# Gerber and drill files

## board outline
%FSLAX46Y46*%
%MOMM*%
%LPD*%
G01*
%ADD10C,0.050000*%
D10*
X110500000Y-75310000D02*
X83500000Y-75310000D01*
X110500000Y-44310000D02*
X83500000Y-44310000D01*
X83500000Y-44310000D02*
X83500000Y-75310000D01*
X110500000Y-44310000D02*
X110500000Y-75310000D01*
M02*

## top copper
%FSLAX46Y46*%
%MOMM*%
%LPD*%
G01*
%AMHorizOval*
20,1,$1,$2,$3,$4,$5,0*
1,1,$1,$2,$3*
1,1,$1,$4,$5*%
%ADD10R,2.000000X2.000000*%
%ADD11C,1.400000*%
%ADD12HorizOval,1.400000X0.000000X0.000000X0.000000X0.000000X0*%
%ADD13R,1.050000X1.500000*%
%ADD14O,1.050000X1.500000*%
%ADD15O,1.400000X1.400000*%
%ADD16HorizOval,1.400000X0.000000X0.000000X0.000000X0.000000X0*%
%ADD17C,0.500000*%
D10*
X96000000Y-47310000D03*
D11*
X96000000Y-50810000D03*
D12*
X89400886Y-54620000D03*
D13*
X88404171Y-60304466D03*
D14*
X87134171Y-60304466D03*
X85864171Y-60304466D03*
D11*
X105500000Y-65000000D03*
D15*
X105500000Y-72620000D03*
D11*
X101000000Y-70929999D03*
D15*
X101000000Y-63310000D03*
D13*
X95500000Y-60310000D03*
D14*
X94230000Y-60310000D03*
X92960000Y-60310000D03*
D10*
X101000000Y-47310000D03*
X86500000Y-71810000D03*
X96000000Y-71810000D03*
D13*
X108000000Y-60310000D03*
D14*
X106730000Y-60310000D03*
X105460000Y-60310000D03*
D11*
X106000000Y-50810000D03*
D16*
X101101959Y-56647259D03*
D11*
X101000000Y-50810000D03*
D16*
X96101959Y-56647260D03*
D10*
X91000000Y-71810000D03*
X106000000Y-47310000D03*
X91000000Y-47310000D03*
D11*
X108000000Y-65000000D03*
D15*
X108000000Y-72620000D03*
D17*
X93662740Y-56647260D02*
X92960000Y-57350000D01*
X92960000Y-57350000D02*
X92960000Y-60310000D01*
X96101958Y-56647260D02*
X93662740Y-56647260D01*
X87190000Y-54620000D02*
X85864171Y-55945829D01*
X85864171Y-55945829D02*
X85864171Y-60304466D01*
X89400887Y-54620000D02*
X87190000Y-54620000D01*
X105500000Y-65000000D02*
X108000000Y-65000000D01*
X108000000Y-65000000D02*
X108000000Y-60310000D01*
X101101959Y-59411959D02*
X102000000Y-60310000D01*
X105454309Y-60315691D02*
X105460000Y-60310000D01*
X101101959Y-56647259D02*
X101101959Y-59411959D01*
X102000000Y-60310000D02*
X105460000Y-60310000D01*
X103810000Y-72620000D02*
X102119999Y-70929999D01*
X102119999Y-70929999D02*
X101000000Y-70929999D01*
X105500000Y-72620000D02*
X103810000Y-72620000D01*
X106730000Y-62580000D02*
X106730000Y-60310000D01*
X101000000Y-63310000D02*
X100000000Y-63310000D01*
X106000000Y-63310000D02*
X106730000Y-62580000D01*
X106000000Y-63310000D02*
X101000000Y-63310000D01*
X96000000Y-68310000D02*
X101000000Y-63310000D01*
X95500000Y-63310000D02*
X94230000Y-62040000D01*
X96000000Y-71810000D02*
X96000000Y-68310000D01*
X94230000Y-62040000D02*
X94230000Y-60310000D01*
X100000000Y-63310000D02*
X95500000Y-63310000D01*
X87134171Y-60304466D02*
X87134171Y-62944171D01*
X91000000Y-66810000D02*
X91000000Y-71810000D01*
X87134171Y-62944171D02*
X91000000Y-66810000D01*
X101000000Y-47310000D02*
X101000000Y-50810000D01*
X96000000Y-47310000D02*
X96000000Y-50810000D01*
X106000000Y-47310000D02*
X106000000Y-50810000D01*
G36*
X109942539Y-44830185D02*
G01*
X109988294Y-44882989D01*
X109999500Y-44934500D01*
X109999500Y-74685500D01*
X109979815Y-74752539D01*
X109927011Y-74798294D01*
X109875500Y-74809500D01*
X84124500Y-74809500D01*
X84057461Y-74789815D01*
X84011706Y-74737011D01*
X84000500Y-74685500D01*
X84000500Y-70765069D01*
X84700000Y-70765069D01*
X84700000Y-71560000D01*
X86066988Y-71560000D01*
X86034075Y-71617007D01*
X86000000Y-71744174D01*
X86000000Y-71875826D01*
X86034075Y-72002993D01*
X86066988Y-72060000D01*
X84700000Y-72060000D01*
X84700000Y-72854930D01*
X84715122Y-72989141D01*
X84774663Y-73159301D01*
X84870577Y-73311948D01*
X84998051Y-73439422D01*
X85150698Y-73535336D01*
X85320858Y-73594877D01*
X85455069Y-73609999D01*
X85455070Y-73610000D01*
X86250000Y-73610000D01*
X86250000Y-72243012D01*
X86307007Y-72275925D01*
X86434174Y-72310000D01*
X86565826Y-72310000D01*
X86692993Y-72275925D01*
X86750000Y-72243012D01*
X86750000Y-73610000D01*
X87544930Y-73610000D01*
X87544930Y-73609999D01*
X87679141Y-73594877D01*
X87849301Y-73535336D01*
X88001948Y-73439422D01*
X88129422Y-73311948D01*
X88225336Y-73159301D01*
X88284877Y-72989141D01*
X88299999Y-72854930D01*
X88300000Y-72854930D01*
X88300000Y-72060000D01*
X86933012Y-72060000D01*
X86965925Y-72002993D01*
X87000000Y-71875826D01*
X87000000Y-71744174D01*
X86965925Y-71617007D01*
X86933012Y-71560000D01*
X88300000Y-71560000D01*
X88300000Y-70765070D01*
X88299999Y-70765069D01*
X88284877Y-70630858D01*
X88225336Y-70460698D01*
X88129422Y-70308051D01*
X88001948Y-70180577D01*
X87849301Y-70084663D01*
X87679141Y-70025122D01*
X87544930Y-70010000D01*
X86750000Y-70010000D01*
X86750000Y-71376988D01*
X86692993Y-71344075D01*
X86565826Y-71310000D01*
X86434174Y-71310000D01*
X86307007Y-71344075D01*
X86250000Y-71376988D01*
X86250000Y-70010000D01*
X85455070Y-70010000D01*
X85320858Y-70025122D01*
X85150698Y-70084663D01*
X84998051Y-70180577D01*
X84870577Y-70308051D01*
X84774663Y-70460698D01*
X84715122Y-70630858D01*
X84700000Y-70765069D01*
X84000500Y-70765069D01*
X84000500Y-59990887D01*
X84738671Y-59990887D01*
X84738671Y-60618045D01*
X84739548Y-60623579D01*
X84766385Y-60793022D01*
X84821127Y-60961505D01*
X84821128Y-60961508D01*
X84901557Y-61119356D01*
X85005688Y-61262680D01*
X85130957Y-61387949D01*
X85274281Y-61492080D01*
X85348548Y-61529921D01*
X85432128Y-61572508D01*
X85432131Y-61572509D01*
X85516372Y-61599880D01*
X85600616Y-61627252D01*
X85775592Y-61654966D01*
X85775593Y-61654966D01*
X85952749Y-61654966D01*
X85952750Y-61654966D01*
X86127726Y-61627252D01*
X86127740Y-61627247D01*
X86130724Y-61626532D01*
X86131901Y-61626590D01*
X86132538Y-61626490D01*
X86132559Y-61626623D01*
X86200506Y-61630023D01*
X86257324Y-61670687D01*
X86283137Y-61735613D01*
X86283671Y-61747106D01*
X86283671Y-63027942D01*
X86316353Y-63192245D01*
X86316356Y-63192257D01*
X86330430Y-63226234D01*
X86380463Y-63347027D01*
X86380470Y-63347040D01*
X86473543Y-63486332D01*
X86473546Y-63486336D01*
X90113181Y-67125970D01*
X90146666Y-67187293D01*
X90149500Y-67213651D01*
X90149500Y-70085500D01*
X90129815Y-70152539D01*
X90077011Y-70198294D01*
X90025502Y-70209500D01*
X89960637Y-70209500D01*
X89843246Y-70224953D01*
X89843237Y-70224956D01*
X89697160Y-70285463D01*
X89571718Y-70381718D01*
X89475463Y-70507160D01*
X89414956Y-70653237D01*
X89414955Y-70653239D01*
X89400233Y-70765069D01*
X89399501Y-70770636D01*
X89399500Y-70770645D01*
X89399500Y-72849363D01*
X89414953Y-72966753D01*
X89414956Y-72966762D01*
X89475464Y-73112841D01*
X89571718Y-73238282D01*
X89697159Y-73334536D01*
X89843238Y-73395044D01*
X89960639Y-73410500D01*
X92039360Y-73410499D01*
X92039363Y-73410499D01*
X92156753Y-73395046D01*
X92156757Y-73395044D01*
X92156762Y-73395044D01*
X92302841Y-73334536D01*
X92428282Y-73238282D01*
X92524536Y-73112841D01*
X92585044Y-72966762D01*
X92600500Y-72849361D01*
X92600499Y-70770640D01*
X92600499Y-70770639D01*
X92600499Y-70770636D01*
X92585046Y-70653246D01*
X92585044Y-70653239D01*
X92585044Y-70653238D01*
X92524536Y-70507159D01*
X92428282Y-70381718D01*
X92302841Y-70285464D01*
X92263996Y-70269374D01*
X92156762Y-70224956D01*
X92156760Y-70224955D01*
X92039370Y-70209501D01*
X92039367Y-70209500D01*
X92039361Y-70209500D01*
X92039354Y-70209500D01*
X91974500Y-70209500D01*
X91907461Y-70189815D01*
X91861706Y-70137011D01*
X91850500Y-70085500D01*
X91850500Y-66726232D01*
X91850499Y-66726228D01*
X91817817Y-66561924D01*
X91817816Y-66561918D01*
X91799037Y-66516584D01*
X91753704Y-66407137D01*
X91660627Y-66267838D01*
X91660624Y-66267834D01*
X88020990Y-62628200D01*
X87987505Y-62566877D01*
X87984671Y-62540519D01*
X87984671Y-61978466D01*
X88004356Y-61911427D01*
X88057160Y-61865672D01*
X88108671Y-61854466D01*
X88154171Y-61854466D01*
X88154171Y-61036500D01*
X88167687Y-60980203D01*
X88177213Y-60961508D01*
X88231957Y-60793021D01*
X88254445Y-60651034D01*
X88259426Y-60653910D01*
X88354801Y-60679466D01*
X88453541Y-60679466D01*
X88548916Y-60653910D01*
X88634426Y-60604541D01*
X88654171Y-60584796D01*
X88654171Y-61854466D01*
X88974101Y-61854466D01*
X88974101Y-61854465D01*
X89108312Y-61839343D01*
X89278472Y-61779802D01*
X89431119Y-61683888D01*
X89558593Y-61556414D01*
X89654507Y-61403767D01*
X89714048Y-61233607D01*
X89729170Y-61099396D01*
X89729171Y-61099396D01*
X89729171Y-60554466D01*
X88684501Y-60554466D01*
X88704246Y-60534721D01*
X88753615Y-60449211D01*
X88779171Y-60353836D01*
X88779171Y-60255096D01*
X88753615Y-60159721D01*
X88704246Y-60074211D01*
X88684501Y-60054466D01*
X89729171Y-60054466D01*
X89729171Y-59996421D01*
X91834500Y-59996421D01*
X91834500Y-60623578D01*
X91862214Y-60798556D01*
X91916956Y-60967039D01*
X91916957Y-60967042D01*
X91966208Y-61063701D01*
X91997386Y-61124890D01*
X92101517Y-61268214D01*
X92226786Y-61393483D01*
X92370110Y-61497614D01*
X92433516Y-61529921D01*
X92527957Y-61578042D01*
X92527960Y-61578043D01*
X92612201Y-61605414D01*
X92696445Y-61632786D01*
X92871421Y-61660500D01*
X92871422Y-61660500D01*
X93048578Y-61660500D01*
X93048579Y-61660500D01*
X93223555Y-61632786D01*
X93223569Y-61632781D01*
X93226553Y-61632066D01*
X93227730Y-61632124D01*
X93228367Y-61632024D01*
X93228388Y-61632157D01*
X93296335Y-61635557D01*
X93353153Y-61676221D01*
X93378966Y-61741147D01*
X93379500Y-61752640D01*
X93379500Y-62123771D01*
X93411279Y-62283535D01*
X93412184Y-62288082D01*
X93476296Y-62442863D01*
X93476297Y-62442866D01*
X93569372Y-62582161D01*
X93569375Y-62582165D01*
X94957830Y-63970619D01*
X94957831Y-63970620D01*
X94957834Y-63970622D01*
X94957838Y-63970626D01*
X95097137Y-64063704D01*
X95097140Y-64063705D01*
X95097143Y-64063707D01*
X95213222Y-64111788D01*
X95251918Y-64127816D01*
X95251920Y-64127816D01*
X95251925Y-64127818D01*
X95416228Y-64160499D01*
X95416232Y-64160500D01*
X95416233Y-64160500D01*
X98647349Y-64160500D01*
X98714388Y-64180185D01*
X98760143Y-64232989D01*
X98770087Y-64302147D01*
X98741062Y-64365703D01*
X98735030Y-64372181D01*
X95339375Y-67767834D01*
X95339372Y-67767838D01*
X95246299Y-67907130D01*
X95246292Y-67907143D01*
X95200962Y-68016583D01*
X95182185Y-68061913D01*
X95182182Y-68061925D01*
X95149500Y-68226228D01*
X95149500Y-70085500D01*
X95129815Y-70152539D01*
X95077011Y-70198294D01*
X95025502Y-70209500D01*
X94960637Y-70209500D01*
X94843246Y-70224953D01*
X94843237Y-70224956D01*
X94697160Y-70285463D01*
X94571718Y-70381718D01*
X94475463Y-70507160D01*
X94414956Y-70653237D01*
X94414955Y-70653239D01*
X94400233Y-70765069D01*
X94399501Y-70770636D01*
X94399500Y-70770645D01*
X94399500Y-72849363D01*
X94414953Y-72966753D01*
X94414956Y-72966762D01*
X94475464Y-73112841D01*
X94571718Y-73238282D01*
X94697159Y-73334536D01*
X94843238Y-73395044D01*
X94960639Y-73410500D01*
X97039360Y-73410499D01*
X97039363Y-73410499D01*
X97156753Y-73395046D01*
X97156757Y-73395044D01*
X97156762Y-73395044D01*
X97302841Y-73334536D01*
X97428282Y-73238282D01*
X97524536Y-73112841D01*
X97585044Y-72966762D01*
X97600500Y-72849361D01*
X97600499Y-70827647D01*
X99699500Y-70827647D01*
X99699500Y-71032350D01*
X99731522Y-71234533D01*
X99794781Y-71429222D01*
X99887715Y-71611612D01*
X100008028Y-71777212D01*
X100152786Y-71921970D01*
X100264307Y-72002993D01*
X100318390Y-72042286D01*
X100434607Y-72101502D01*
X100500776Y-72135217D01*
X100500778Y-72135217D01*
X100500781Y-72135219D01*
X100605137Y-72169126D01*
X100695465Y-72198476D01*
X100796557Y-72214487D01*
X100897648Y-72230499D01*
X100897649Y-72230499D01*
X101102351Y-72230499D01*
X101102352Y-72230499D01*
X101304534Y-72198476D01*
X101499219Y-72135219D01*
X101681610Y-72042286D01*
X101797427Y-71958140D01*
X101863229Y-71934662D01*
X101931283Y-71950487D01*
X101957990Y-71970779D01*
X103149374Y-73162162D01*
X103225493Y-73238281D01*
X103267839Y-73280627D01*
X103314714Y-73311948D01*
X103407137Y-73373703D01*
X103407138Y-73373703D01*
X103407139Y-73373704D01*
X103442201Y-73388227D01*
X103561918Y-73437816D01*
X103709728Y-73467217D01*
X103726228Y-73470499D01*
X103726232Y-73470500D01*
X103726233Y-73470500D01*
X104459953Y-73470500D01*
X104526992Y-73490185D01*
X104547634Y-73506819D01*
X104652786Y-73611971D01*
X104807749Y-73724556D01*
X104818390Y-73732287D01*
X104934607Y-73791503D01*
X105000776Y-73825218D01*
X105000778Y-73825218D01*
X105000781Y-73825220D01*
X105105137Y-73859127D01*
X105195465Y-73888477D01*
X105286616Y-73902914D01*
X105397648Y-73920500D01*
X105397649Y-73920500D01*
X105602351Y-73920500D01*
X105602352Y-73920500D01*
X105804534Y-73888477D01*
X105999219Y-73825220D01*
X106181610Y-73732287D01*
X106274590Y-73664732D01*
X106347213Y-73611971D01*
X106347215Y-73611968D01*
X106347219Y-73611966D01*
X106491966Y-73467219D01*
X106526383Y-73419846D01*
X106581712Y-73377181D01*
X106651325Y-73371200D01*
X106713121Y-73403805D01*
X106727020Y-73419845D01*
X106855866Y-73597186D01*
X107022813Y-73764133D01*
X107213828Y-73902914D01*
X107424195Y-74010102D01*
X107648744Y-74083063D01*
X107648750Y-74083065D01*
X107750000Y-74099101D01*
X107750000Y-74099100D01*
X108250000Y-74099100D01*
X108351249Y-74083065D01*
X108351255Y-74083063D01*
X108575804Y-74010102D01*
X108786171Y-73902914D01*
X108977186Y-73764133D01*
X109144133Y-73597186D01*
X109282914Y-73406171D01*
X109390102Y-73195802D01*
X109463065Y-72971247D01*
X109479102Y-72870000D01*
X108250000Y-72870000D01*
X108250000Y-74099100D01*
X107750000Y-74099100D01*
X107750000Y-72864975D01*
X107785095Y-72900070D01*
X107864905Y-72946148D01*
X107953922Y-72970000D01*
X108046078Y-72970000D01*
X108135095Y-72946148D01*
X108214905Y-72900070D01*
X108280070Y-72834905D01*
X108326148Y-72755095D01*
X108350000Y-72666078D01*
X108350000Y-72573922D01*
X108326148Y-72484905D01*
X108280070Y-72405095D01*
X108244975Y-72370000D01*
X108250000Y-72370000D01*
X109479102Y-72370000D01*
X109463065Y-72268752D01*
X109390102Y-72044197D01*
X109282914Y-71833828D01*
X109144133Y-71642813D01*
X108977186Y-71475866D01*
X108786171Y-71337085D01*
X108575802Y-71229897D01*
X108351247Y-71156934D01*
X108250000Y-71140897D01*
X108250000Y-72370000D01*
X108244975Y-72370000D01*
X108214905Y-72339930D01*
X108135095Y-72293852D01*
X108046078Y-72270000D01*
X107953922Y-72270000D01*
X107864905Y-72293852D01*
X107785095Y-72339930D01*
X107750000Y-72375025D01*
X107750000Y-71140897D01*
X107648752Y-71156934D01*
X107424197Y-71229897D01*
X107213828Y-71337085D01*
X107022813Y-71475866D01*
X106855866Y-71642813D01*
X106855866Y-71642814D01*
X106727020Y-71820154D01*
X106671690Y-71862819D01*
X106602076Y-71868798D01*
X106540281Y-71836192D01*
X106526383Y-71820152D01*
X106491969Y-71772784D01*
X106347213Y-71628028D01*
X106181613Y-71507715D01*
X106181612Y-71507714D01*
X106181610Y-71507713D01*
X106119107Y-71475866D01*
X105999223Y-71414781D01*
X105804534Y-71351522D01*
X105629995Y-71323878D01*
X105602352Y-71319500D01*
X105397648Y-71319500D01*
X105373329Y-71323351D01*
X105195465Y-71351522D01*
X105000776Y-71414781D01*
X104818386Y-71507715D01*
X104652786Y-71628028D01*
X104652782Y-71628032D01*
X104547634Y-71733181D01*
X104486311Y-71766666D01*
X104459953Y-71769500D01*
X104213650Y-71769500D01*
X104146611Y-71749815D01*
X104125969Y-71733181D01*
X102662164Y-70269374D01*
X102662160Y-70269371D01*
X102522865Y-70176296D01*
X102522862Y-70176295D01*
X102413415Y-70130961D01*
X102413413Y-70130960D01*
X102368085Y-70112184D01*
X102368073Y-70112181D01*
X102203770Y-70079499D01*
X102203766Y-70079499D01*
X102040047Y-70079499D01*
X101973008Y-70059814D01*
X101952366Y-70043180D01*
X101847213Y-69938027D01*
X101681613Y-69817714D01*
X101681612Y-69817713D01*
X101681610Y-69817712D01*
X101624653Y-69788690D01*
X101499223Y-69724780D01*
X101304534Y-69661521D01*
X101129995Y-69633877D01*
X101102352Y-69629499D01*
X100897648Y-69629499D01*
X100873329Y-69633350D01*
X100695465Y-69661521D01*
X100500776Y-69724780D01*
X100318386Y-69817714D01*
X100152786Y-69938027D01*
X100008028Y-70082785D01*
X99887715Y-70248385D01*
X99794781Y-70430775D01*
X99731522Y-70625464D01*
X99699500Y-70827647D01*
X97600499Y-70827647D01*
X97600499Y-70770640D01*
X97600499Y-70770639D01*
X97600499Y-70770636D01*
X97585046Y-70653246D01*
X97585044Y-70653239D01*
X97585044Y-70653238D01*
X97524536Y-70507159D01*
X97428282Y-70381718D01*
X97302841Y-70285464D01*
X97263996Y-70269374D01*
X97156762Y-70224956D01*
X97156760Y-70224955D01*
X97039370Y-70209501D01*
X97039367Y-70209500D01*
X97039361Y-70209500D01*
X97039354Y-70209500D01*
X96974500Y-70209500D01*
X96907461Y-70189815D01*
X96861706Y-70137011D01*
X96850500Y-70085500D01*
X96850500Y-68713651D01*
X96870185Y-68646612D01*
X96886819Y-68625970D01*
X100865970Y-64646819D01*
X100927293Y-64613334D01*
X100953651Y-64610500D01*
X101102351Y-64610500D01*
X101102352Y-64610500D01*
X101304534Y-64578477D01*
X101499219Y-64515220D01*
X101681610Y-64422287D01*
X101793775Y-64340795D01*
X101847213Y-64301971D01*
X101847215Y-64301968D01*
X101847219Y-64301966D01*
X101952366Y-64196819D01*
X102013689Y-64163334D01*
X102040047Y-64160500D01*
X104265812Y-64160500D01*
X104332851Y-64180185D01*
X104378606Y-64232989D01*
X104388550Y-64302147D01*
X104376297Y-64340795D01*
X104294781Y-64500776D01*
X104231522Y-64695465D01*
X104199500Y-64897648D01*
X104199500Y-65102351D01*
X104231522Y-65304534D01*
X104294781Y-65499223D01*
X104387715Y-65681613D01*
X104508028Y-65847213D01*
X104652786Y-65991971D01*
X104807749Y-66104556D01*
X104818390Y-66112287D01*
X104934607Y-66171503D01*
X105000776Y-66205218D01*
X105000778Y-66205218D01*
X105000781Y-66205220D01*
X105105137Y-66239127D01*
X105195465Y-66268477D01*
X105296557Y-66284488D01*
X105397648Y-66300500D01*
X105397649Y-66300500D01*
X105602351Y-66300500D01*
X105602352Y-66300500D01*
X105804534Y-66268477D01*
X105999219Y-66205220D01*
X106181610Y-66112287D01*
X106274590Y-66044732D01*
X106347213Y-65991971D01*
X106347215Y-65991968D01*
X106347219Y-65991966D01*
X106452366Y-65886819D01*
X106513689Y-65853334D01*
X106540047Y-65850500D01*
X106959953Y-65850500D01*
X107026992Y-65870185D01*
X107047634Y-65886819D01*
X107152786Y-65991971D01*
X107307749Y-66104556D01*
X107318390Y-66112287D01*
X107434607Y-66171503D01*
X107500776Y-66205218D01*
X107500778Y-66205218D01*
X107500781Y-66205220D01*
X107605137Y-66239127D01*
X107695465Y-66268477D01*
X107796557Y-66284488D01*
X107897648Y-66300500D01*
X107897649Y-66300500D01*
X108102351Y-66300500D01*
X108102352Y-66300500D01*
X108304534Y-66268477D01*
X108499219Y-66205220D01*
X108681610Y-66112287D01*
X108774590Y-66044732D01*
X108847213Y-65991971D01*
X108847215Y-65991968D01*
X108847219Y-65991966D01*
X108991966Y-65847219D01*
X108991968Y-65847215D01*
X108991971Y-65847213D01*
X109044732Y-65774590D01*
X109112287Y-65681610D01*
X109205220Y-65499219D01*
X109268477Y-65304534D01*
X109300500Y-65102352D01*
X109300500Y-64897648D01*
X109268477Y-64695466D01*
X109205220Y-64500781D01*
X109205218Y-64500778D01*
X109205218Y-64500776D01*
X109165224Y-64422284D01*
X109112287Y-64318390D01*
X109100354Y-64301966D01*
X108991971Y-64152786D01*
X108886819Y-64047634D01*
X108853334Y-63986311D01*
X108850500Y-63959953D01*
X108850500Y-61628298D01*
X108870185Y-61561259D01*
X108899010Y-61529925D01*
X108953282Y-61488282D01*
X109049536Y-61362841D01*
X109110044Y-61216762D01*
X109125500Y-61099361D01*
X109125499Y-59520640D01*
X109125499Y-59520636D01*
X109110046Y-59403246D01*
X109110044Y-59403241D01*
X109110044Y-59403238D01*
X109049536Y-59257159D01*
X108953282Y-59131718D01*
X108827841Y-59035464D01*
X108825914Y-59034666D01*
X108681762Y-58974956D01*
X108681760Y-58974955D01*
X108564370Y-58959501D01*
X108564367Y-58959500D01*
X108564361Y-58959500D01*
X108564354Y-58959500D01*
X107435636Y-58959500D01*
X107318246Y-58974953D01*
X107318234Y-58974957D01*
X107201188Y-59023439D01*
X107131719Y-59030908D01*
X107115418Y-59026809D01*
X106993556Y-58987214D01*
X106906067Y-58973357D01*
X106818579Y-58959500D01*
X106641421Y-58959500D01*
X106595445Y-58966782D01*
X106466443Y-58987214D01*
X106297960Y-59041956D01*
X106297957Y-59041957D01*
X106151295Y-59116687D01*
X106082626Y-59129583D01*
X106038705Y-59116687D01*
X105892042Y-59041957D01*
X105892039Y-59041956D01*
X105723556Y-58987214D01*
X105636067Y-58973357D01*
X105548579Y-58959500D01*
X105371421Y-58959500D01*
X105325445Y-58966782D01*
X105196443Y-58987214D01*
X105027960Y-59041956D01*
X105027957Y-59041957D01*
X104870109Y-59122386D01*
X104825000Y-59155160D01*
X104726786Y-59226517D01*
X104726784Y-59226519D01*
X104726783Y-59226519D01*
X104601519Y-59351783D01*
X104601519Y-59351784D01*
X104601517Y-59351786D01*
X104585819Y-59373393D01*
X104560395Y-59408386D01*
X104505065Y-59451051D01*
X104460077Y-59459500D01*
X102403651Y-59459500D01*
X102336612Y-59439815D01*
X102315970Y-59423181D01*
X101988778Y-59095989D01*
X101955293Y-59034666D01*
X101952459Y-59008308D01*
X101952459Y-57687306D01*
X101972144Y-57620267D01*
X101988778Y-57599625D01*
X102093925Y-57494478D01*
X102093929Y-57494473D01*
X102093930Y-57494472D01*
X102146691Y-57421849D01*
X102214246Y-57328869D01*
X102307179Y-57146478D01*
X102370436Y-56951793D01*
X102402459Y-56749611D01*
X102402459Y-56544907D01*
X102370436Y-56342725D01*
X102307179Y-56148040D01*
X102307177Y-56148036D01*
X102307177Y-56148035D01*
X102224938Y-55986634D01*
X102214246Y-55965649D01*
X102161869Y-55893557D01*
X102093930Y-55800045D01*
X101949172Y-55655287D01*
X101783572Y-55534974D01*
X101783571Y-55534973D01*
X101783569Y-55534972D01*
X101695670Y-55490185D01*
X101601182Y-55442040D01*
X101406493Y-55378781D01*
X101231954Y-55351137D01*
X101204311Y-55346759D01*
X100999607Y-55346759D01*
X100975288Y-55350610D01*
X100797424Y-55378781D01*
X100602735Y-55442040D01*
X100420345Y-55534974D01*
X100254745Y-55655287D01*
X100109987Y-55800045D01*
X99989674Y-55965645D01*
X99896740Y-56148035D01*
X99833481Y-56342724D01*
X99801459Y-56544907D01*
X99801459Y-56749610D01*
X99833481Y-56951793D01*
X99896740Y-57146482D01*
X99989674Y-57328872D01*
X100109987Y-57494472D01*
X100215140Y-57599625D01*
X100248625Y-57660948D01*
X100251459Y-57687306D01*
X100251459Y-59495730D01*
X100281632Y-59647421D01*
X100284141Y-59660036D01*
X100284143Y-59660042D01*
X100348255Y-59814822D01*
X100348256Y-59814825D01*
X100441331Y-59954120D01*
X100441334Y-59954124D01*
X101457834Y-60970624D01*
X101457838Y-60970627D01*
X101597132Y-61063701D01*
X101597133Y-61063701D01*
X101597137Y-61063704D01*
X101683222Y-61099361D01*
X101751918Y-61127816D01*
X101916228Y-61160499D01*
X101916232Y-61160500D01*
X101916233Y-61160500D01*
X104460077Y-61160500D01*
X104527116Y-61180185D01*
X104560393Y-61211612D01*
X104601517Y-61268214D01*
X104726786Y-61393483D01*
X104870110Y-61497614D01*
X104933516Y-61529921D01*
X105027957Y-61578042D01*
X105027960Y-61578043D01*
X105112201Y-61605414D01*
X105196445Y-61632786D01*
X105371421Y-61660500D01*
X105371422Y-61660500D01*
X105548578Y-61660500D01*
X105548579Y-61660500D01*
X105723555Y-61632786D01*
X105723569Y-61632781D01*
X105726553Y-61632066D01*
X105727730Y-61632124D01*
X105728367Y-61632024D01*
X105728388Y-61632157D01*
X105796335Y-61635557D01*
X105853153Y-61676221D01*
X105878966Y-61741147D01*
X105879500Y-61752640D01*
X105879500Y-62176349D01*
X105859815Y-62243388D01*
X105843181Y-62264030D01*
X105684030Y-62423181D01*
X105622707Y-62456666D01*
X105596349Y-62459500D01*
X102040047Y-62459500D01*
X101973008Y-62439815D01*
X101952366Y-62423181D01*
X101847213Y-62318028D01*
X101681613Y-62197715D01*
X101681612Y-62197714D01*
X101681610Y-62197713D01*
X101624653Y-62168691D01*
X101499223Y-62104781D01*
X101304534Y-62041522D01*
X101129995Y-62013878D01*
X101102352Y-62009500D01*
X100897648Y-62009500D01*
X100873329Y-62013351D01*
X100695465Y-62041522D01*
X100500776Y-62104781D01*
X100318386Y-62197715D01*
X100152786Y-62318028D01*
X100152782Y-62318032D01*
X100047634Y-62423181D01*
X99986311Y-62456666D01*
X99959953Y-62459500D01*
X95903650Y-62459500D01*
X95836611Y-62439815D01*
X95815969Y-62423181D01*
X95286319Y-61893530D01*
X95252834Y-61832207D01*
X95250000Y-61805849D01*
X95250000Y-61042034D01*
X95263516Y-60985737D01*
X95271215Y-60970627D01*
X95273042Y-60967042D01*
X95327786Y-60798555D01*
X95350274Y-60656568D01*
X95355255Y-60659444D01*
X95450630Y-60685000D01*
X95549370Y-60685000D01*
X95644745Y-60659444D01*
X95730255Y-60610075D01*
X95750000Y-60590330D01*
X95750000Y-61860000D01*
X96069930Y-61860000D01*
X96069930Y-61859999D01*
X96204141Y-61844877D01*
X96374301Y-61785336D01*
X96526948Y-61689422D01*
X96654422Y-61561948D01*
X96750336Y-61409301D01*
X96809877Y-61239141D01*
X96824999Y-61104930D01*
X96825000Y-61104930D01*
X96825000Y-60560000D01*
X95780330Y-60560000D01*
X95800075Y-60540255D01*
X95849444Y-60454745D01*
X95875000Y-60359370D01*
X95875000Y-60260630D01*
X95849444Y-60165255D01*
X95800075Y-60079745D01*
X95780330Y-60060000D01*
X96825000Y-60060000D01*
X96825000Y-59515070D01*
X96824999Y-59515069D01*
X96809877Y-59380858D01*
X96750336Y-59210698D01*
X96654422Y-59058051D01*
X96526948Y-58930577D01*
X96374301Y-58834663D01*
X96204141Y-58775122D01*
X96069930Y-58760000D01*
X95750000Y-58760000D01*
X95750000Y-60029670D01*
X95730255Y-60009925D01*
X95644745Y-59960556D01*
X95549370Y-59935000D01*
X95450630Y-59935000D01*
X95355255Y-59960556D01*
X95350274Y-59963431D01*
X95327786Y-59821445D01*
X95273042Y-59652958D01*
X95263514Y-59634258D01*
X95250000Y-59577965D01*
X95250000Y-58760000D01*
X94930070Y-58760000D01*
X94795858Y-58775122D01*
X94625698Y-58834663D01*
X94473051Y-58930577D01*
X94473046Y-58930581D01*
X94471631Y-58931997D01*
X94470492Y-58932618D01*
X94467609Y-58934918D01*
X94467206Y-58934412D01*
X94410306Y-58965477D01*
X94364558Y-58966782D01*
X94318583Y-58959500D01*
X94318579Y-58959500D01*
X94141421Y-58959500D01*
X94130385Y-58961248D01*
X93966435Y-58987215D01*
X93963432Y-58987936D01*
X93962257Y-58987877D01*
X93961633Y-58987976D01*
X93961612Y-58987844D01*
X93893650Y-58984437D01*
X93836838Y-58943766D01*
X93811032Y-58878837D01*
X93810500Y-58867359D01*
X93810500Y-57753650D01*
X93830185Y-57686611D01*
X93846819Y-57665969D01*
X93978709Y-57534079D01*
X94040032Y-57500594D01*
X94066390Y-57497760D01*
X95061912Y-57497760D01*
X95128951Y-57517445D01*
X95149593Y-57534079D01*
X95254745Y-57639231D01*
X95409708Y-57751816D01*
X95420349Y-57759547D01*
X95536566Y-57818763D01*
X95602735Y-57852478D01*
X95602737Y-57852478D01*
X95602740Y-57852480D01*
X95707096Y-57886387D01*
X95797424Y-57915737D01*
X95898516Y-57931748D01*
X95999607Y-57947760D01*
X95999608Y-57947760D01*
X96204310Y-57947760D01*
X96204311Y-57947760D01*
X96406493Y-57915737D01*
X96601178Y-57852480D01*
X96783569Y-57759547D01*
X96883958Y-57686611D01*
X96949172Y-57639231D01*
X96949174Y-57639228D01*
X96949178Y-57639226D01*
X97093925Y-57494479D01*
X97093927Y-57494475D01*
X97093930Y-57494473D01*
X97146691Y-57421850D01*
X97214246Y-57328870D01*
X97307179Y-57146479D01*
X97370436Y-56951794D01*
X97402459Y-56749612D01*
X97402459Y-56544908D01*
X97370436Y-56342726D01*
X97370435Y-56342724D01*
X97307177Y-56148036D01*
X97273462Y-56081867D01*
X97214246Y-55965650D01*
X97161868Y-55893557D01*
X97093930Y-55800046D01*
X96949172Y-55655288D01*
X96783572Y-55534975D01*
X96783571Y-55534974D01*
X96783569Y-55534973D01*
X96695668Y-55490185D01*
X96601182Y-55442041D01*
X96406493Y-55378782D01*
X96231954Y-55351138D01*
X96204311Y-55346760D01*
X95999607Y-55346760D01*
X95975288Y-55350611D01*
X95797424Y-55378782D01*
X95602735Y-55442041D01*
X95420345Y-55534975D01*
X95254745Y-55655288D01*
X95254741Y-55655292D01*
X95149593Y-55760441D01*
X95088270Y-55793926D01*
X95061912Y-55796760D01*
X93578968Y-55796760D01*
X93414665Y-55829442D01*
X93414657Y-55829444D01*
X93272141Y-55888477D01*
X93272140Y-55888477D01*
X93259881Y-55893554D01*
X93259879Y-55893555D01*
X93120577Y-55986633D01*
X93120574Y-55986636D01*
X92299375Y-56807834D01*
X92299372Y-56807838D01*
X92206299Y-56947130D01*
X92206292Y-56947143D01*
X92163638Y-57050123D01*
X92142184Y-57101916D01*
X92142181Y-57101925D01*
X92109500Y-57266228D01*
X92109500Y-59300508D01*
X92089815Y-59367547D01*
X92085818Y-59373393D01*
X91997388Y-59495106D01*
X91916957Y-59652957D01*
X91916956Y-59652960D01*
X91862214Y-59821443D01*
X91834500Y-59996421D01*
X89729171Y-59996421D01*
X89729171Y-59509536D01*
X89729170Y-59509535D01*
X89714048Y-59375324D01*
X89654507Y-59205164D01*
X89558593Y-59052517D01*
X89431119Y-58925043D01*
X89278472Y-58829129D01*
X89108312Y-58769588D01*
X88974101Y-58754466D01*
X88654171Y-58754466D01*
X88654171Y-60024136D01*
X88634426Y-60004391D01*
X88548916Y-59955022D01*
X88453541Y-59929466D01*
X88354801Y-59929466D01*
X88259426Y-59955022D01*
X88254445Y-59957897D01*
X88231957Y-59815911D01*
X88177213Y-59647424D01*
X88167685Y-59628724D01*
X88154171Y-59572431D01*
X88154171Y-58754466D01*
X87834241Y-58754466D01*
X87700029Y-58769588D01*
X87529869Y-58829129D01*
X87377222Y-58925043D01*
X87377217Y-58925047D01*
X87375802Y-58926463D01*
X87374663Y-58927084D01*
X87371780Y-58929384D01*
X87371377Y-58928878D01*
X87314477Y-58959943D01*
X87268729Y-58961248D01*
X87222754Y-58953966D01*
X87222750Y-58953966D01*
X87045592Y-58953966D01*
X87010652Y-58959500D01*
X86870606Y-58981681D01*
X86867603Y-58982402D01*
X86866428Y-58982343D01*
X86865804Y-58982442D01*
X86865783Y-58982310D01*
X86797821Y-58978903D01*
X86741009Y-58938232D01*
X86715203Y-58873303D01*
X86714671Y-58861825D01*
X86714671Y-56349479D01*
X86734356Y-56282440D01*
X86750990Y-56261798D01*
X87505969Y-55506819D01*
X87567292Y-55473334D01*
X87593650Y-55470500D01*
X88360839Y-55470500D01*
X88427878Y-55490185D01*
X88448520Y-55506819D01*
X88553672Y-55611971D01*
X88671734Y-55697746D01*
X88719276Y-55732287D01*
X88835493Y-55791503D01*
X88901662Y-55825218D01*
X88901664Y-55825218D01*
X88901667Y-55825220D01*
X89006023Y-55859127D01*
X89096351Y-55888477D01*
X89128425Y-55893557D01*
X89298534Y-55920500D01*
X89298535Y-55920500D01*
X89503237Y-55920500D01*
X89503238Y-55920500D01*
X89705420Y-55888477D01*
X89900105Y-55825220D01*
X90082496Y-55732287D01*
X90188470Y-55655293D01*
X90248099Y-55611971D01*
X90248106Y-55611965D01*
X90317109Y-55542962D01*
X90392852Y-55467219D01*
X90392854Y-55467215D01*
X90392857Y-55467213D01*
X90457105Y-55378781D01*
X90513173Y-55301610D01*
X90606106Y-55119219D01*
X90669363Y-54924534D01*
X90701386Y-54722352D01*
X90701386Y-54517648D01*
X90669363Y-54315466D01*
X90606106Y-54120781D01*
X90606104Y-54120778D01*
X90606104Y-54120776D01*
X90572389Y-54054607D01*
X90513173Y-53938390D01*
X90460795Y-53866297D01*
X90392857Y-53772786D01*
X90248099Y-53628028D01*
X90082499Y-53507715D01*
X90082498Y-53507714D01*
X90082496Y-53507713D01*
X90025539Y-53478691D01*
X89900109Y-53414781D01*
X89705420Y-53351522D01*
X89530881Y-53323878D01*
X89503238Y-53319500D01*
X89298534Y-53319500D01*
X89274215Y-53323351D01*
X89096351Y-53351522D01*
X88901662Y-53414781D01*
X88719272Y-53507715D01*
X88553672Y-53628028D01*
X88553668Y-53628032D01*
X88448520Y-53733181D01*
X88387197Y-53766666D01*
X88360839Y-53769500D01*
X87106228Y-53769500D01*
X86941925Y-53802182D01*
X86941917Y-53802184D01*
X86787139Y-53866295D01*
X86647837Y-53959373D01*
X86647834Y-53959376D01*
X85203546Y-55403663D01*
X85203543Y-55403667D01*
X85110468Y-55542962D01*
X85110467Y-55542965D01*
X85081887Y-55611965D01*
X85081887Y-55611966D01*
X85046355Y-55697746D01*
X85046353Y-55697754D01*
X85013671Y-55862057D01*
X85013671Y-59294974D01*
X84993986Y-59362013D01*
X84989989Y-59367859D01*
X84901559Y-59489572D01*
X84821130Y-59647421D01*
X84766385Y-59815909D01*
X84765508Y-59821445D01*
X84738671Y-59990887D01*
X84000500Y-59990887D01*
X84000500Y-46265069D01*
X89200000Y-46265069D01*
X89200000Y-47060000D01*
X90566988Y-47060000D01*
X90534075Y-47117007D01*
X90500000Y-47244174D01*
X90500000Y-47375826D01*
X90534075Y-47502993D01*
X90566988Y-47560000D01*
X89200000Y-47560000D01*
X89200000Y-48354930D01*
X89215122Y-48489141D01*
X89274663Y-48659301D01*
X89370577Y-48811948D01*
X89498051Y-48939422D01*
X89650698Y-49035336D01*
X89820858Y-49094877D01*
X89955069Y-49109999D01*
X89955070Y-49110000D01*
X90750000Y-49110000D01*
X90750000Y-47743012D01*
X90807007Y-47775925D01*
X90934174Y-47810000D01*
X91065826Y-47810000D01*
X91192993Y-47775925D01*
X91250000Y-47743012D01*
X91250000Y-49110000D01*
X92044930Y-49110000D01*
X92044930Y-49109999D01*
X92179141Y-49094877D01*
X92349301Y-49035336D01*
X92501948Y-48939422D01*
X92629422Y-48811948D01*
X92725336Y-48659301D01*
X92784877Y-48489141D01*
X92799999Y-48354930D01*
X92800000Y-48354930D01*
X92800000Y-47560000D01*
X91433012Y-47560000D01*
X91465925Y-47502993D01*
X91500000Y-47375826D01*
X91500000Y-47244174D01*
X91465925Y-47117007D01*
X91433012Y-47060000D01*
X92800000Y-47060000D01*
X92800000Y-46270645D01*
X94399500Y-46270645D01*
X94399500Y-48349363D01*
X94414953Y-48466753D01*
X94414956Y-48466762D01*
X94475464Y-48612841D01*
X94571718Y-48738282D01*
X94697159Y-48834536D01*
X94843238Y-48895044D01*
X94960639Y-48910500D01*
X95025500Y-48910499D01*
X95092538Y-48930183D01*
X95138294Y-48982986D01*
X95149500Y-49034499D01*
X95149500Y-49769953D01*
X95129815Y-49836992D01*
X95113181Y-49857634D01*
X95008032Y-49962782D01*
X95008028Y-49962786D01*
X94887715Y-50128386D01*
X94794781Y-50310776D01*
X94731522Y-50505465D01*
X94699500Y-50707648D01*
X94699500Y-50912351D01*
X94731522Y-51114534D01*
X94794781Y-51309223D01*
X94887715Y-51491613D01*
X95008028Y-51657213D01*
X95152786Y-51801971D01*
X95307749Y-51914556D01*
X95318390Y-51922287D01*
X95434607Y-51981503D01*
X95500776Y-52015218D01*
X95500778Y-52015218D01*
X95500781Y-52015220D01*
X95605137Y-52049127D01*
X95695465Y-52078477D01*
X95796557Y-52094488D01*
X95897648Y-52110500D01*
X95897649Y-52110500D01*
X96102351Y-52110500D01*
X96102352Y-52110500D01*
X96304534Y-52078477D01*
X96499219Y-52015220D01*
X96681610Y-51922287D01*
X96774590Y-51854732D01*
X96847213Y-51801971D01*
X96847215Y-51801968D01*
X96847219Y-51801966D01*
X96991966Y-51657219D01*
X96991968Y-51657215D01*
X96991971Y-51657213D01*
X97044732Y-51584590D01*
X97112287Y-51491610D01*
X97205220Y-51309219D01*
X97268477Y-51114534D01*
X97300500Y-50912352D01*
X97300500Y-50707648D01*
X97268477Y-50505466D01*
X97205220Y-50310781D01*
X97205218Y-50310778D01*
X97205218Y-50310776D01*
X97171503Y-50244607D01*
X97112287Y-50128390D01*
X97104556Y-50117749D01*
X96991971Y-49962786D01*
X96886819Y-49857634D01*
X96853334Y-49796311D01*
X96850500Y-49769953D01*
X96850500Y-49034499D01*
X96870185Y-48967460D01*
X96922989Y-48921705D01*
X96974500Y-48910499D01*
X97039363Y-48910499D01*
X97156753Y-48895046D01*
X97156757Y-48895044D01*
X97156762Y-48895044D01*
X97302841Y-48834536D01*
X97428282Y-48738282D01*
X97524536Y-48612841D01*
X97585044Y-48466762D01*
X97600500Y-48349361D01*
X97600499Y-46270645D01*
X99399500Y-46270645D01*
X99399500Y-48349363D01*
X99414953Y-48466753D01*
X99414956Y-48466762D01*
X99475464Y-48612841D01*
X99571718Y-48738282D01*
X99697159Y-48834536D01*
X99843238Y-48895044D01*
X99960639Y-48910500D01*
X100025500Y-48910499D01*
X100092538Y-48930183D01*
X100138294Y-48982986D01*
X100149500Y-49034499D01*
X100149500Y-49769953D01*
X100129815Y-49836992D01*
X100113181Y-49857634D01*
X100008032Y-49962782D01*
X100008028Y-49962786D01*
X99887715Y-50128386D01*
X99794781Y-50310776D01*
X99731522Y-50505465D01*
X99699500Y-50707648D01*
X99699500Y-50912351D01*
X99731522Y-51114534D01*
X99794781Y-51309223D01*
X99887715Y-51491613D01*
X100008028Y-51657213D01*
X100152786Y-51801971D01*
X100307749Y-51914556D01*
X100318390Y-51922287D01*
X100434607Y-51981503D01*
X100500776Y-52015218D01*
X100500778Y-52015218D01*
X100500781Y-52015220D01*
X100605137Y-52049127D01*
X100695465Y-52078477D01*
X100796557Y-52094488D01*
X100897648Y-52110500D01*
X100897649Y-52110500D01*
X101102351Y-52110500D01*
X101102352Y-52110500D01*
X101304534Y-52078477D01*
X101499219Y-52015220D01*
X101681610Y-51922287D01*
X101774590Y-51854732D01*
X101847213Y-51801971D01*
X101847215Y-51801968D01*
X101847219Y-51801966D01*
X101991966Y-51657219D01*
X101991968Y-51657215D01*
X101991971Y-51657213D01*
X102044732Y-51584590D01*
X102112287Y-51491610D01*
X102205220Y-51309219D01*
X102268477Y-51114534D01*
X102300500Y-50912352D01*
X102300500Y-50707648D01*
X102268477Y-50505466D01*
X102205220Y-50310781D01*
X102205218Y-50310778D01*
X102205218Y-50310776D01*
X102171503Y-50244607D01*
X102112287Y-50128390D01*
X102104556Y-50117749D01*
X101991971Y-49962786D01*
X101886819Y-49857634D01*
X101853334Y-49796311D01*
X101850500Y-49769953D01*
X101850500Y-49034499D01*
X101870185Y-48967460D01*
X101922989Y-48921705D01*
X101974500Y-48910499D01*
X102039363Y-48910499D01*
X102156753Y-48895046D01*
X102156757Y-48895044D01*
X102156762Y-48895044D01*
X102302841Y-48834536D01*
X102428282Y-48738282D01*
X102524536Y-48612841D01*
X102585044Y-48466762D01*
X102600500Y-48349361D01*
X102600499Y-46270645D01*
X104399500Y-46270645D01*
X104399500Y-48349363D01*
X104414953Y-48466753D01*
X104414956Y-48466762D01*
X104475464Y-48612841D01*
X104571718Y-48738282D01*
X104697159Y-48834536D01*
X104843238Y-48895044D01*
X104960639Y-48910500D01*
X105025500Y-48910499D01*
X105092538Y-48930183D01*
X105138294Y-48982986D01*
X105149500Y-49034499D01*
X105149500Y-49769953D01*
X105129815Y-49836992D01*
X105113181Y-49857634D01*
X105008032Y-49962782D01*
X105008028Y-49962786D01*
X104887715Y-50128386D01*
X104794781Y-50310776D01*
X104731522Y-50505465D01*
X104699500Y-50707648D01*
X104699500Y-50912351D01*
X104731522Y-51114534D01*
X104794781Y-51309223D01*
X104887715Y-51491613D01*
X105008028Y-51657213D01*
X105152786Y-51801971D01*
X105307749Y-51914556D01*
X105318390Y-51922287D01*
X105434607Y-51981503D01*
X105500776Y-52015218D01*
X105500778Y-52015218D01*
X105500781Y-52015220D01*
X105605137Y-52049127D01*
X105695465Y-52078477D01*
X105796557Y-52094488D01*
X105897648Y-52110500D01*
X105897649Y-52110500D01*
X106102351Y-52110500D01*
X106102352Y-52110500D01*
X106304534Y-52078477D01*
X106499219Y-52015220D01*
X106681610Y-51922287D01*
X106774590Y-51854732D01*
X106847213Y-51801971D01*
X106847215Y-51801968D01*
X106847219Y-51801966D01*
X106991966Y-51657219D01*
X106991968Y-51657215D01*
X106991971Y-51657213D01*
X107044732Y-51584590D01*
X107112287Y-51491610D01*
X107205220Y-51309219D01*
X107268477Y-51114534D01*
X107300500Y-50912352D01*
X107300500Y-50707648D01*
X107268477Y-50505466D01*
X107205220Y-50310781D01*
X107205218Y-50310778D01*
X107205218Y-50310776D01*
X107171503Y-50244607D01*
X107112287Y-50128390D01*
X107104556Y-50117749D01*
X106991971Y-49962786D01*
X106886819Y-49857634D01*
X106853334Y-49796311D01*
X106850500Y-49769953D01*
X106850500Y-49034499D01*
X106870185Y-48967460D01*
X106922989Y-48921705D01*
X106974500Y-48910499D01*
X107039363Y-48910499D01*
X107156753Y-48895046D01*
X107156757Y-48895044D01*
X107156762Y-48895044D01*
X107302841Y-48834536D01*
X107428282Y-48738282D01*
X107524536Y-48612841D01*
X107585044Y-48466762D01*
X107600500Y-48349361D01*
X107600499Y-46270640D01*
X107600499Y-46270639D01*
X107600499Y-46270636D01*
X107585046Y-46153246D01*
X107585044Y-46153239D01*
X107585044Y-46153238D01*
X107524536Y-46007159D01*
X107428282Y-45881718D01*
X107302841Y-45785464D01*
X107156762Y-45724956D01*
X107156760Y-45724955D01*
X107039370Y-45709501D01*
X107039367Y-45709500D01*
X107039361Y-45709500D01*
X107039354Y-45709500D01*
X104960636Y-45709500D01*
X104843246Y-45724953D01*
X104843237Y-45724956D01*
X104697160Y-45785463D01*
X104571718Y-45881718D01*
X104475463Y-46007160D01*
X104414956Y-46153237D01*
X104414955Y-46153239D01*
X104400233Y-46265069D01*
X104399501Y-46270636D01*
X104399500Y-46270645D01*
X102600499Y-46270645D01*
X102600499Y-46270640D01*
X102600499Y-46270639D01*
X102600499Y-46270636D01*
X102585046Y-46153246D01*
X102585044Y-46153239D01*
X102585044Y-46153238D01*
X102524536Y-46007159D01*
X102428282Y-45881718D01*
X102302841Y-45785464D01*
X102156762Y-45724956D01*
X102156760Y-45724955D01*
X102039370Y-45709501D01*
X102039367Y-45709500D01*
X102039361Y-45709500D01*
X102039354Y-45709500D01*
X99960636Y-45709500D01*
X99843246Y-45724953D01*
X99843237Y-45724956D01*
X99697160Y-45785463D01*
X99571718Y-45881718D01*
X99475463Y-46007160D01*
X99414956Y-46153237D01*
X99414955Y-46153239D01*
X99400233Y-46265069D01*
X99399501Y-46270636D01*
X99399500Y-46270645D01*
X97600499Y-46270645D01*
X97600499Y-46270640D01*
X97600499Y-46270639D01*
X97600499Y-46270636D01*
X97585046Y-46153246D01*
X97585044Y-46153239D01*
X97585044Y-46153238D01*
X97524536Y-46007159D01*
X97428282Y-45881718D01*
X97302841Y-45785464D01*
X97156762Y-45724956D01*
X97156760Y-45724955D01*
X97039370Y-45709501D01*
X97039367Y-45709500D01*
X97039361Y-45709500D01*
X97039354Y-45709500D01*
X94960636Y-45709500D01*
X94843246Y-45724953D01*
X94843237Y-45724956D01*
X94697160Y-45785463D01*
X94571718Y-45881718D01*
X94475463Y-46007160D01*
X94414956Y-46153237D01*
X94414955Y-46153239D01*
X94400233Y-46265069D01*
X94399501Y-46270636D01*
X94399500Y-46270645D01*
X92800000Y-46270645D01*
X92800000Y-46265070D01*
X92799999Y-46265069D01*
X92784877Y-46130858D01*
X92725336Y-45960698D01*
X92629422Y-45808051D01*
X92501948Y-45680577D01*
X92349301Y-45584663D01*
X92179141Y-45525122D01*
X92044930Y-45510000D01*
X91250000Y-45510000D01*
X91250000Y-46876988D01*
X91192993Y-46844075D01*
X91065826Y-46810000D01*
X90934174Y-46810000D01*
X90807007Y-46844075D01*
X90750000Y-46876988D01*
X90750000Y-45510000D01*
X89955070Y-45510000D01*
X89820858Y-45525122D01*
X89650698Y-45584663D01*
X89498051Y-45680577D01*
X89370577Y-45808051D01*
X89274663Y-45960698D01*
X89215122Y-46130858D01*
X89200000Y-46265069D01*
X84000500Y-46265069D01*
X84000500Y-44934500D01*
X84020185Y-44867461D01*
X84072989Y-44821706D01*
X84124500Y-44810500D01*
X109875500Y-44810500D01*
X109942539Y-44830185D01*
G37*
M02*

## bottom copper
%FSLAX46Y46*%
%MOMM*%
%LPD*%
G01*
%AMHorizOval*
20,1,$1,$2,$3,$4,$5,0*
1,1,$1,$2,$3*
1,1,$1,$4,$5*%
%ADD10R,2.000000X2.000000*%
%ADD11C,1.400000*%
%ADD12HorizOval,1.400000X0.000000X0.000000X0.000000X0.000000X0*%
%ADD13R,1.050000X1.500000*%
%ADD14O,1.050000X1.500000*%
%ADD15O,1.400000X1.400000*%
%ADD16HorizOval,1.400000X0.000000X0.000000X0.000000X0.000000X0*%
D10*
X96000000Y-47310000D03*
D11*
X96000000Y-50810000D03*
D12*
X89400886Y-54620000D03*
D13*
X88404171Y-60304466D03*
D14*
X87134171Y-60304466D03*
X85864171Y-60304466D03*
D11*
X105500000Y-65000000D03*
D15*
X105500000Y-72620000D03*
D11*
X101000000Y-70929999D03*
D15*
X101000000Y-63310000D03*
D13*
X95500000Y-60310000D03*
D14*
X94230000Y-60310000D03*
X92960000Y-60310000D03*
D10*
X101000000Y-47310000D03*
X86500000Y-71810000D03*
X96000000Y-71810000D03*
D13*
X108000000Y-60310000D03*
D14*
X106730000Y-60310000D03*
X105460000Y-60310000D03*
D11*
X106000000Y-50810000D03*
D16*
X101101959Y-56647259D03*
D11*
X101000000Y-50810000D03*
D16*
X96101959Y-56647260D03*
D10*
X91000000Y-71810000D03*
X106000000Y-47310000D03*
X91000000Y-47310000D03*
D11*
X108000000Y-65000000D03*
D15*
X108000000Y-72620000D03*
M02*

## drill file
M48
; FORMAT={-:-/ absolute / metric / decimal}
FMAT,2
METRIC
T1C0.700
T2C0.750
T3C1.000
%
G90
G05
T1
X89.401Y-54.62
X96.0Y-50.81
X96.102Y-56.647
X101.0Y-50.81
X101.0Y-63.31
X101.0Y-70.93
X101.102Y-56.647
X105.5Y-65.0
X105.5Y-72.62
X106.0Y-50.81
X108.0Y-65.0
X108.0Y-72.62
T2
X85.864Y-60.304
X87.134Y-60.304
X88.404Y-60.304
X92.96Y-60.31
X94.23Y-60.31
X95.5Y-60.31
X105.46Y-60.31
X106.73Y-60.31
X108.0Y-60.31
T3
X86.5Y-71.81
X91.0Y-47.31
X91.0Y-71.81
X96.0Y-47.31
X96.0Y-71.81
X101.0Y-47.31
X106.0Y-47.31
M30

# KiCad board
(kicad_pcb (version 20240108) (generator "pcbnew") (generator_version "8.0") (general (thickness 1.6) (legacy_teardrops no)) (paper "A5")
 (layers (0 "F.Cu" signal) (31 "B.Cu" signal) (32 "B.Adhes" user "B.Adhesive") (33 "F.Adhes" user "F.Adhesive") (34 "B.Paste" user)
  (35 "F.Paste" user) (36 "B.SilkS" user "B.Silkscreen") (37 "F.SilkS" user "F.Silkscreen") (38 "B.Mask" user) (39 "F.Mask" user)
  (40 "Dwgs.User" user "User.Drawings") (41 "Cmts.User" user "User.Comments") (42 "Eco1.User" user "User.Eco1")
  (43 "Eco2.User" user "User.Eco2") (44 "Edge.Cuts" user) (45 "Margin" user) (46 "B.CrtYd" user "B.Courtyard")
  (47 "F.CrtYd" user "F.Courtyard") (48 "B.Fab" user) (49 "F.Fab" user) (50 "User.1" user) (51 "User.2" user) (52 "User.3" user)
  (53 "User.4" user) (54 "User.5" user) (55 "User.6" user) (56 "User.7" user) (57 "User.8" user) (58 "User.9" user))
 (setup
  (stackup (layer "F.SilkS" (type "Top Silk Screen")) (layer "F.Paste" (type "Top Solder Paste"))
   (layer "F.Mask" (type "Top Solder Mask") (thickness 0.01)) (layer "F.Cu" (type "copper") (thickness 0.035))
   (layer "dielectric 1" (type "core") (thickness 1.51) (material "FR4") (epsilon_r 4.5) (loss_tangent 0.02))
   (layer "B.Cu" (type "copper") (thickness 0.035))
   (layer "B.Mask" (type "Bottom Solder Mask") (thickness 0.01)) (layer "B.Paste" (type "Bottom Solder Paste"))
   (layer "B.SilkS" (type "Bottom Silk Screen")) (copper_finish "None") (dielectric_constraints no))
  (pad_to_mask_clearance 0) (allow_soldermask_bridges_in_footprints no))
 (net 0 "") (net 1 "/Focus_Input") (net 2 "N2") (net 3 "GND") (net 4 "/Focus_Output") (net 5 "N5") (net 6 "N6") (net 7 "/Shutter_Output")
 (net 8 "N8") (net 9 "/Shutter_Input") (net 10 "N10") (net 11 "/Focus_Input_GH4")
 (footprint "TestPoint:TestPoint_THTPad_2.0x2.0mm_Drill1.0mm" (layer "F.Cu") (at 96 47.31)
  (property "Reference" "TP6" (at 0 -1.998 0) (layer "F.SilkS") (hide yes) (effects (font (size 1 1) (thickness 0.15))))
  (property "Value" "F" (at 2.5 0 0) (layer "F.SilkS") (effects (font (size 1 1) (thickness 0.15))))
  (pad "1" thru_hole rect (at 0 0) (size 2 2) (drill 1) (layers "*.Cu" "*.Mask") (remove_unused_layers no) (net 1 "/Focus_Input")))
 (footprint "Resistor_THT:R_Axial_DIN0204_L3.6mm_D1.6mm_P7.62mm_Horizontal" (layer "F.Cu") (at 96 50.81 -150)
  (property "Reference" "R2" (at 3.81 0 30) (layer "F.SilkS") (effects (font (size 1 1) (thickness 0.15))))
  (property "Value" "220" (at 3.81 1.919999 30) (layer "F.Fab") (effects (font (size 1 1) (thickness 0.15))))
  (pad "1" thru_hole circle (at 0 0 210) (size 1.4 1.4) (drill 0.7) (layers "*.Cu" "*.Mask") (remove_unused_layers no)
   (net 1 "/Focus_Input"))
  (pad "2" thru_hole oval (at 7.62 0 210) (size 1.4 1.4) (drill 0.7) (layers "*.Cu" "*.Mask") (remove_unused_layers no) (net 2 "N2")))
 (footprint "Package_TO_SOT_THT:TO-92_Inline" (layer "F.Cu") (at 88.404171 60.304466 180)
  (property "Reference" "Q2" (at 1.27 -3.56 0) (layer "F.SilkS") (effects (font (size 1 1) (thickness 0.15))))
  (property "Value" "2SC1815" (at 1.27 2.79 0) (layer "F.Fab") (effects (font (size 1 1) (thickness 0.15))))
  (pad "1" thru_hole rect (at 0 0 180) (size 1.05 1.5) (drill 0.75) (layers "*.Cu" "*.Mask") (remove_unused_layers no) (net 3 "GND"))
  (pad "2" thru_hole oval (at 1.27 0 180) (size 1.05 1.5) (drill 0.75) (layers "*.Cu" "*.Mask") (remove_unused_layers no)
   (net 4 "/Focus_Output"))
  (pad "3" thru_hole oval (at 2.54 0 180) (size 1.05 1.5) (drill 0.75) (layers "*.Cu" "*.Mask") (remove_unused_layers no) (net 2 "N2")))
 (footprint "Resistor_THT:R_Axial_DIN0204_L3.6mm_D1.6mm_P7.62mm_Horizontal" (layer "F.Cu") (at 105.5 65 -90)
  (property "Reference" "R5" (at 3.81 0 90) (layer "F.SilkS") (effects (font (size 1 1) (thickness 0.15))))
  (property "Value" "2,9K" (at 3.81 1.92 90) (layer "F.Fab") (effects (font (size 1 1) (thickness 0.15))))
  (pad "1" thru_hole circle (at 0 0 270) (size 1.4 1.4) (drill 0.7) (layers "*.Cu" "*.Mask") (remove_unused_layers no) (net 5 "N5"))
  (pad "2" thru_hole oval (at 7.62 0 270) (size 1.4 1.4) (drill 0.7) (layers "*.Cu" "*.Mask") (remove_unused_layers no) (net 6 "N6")))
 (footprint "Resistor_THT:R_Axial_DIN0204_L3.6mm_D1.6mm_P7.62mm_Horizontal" (layer "F.Cu") (at 101 70.929999 90)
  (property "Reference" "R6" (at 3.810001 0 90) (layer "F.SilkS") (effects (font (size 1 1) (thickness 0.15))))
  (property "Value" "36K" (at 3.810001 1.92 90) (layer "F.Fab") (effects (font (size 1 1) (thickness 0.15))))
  (pad "1" thru_hole circle (at 0 0 90) (size 1.4 1.4) (drill 0.7) (layers "*.Cu" "*.Mask") (remove_unused_layers no) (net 6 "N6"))
  (pad "2" thru_hole oval (at 7.619999 0 90) (size 1.4 1.4) (drill 0.7) (layers "*.Cu" "*.Mask") (remove_unused_layers no)
   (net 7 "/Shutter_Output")))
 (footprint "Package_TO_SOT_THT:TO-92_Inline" (layer "F.Cu") (at 95.5 60.31 180)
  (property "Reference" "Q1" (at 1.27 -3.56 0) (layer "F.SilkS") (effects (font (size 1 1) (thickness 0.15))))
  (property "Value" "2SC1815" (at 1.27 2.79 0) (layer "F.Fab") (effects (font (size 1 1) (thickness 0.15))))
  (pad "1" thru_hole rect (at 0 0 180) (size 1.05 1.5) (drill 0.75) (layers "*.Cu" "*.Mask") (remove_unused_layers no) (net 3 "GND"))
  (pad "2" thru_hole oval (at 1.27 0 180) (size 1.05 1.5) (drill 0.75) (layers "*.Cu" "*.Mask") (remove_unused_layers no)
   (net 7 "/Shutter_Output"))
  (pad "3" thru_hole oval (at 2.54 0 180) (size 1.05 1.5) (drill 0.75) (layers "*.Cu" "*.Mask") (remove_unused_layers no) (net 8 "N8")))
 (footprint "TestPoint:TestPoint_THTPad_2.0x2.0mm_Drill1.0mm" (layer "F.Cu") (at 101 47.31)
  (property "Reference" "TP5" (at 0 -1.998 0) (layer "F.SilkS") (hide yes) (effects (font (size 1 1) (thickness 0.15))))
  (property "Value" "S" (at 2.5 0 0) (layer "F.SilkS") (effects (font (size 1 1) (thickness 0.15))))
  (pad "1" thru_hole rect (at 0 0) (size 2 2) (drill 1) (layers "*.Cu" "*.Mask") (remove_unused_layers no) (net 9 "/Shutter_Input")))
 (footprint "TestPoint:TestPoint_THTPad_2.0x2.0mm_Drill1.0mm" (layer "F.Cu") (at 86.5 71.81)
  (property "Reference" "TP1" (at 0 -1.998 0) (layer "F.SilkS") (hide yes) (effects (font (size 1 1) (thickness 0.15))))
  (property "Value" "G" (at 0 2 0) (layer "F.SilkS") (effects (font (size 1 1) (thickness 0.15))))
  (pad "1" thru_hole rect (at 0 0) (size 2 2) (drill 1) (layers "*.Cu" "*.Mask") (remove_unused_layers no) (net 3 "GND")))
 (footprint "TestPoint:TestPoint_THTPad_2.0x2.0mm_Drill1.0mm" (layer "F.Cu") (at 96 71.81)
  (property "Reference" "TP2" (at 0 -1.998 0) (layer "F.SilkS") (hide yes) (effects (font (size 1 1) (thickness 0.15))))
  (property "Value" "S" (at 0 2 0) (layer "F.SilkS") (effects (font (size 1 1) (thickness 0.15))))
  (pad "1" thru_hole rect (at 0 0) (size 2 2) (drill 1) (layers "*.Cu" "*.Mask") (remove_unused_layers no) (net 7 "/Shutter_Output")))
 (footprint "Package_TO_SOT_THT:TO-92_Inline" (layer "F.Cu") (at 108 60.31 180)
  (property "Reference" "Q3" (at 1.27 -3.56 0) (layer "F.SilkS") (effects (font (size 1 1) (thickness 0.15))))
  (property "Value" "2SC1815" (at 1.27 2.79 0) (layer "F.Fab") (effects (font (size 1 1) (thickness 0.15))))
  (pad "1" thru_hole rect (at 0 0 180) (size 1.05 1.5) (drill 0.75) (layers "*.Cu" "*.Mask") (remove_unused_layers no) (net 5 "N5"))
  (pad "2" thru_hole oval (at 1.27 0 180) (size 1.05 1.5) (drill 0.75) (layers "*.Cu" "*.Mask") (remove_unused_layers no)
   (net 7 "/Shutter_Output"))
  (pad "3" thru_hole oval (at 2.54 0 180) (size 1.05 1.5) (drill 0.75) (layers "*.Cu" "*.Mask") (remove_unused_layers no) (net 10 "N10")))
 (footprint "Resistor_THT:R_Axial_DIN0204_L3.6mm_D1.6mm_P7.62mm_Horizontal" (layer "F.Cu") (at 106 50.81 -130)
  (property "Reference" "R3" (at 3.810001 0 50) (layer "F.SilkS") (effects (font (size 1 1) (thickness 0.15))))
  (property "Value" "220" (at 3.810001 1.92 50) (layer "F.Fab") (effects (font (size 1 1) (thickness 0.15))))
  (pad "1" thru_hole circle (at 0 0 230) (size 1.4 1.4) (drill 0.7) (layers "*.Cu" "*.Mask") (remove_unused_layers no)
   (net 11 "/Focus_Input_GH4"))
  (pad "2" thru_hole oval (at 7.62 -0.000001 230) (size 1.4 1.4) (drill 0.7) (layers "*.Cu" "*.Mask") (remove_unused_layers no)
   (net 10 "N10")))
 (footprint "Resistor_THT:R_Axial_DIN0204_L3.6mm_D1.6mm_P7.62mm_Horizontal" (layer "F.Cu") (at 101 50.81 -130)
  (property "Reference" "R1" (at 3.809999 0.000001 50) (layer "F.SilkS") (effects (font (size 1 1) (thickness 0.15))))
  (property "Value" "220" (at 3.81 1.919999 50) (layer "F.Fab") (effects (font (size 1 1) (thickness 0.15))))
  (pad "1" thru_hole circle (at 0 0 230) (size 1.4 1.4) (drill 0.7) (layers "*.Cu" "*.Mask") (remove_unused_layers no)
   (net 9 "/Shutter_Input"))
  (pad "2" thru_hole oval (at 7.620001 -0.000001 230) (size 1.4 1.4) (drill 0.7) (layers "*.Cu" "*.Mask") (remove_unused_layers no)
   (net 8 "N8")))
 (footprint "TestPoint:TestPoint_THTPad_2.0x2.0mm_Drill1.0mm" (layer "F.Cu") (at 91 71.81)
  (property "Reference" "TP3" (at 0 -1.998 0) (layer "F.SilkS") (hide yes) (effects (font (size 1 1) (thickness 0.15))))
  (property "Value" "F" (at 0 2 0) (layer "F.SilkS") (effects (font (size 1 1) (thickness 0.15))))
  (pad "1" thru_hole rect (at 0 0) (size 2 2) (drill 1) (layers "*.Cu" "*.Mask") (remove_unused_layers no) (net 4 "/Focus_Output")))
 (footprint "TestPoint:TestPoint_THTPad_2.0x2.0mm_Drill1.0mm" (layer "F.Cu") (at 106 47.31)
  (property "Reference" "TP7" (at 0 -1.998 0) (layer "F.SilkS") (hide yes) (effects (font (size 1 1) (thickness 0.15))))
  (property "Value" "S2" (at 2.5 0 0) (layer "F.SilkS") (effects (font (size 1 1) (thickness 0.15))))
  (pad "1" thru_hole rect (at 0 0) (size 2 2) (drill 1) (layers "*.Cu" "*.Mask") (remove_unused_layers no) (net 11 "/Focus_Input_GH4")))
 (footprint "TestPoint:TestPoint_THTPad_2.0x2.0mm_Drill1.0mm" (layer "F.Cu") (at 91 47.31)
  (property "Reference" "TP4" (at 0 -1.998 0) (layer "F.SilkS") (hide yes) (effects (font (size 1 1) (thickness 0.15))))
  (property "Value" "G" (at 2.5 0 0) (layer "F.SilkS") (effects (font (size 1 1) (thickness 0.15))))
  (pad "1" thru_hole rect (at 0 0) (size 2 2) (drill 1) (layers "*.Cu" "*.Mask") (remove_unused_layers no) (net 3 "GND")))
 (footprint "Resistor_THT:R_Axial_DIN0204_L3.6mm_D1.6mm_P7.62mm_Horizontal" (layer "F.Cu") (at 108 65 -90)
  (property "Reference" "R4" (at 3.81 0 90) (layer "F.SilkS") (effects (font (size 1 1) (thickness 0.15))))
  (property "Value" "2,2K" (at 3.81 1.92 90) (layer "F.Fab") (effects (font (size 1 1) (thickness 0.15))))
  (pad "1" thru_hole circle (at 0 0 270) (size 1.4 1.4) (drill 0.7) (layers "*.Cu" "*.Mask") (remove_unused_layers no) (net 5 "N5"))
  (pad "2" thru_hole oval (at 7.62 0 270) (size 1.4 1.4) (drill 0.7) (layers "*.Cu" "*.Mask") (remove_unused_layers no) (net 3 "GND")))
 (gr_line (start 110.5 75.31) (end 83.5 75.31) (stroke (width 0.05) (type default)) (layer "Edge.Cuts"))
 (gr_line (start 110.5 44.31) (end 83.5 44.31) (stroke (width 0.05) (type default)) (layer "Edge.Cuts"))
 (gr_line (start 83.5 44.31) (end 83.5 75.31) (stroke (width 0.05) (type default)) (layer "Edge.Cuts"))
 (gr_line (start 110.5 44.31) (end 110.5 75.31) (stroke (width 0.05) (type default)) (layer "Edge.Cuts"))
 (segment (start 93.66274 56.64726) (end 92.96 57.35) (width 0.5) (layer "F.Cu") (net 8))
 (segment (start 92.96 57.35) (end 92.96 60.31) (width 0.5) (layer "F.Cu") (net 8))
 (segment (start 96.101958 56.64726) (end 93.66274 56.64726) (width 0.5) (layer "F.Cu") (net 8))
 (segment (start 87.19 54.62) (end 85.864171 55.945829) (width 0.5) (layer "F.Cu") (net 2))
 (segment (start 85.864171 55.945829) (end 85.864171 60.304466) (width 0.5) (layer "F.Cu") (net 2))
 (segment (start 89.400887 54.62) (end 87.19 54.62) (width 0.5) (layer "F.Cu") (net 2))
 (segment (start 105.5 65) (end 108 65) (width 0.5) (layer "F.Cu") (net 5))
 (segment (start 108 65) (end 108 60.31) (width 0.5) (layer "F.Cu") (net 5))
 (segment (start 101.101959 59.411959) (end 102 60.31) (width 0.5) (layer "F.Cu") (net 10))
 (segment (start 105.454309 60.315691) (end 105.46 60.31) (width 0.5) (layer "F.Cu") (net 10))
 (segment (start 101.101959 56.647259) (end 101.101959 59.411959) (width 0.5) (layer "F.Cu") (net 10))
 (segment (start 102 60.31) (end 105.46 60.31) (width 0.5) (layer "F.Cu") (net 10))
 (segment (start 103.81 72.62) (end 102.119999 70.929999) (width 0.5) (layer "F.Cu") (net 6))
 (segment (start 102.119999 70.929999) (end 101 70.929999) (width 0.5) (layer "F.Cu") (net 6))
 (segment (start 105.5 72.62) (end 103.81 72.62) (width 0.5) (layer "F.Cu") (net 6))
 (segment (start 106.73 62.58) (end 106.73 60.31) (width 0.5) (layer "F.Cu") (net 7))
 (segment (start 101 63.31) (end 100 63.31) (width 0.5) (layer "F.Cu") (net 7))
 (segment (start 106 63.31) (end 106.73 62.58) (width 0.5) (layer "F.Cu") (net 7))
 (segment (start 106 63.31) (end 101 63.31) (width 0.5) (layer "F.Cu") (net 7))
 (segment (start 96 68.31) (end 101 63.31) (width 0.5) (layer "F.Cu") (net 7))
 (segment (start 95.5 63.31) (end 94.23 62.04) (width 0.5) (layer "F.Cu") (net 7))
 (segment (start 96 71.81) (end 96 68.31) (width 0.5) (layer "F.Cu") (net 7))
 (segment (start 94.23 62.04) (end 94.23 60.31) (width 0.5) (layer "F.Cu") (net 7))
 (segment (start 100 63.31) (end 95.5 63.31) (width 0.5) (layer "F.Cu") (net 7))
 (segment (start 87.134171 60.304466) (end 87.134171 62.944171) (width 0.5) (layer "F.Cu") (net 4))
 (segment (start 91 66.81) (end 91 71.81) (width 0.5) (layer "F.Cu") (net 4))
 (segment (start 87.134171 62.944171) (end 91 66.81) (width 0.5) (layer "F.Cu") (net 4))
 (segment (start 101 47.31) (end 101 50.81) (width 0.5) (layer "F.Cu") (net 9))
 (segment (start 96 47.31) (end 96 50.81) (width 0.5) (layer "F.Cu") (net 1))
 (segment (start 106 47.31) (end 106 50.81) (width 0.5) (layer "F.Cu") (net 11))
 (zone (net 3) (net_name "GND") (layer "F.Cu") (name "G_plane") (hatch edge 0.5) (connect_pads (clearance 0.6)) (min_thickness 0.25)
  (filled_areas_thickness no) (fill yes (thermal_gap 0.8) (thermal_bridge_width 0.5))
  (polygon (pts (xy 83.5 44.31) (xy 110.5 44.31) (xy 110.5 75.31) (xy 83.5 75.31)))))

